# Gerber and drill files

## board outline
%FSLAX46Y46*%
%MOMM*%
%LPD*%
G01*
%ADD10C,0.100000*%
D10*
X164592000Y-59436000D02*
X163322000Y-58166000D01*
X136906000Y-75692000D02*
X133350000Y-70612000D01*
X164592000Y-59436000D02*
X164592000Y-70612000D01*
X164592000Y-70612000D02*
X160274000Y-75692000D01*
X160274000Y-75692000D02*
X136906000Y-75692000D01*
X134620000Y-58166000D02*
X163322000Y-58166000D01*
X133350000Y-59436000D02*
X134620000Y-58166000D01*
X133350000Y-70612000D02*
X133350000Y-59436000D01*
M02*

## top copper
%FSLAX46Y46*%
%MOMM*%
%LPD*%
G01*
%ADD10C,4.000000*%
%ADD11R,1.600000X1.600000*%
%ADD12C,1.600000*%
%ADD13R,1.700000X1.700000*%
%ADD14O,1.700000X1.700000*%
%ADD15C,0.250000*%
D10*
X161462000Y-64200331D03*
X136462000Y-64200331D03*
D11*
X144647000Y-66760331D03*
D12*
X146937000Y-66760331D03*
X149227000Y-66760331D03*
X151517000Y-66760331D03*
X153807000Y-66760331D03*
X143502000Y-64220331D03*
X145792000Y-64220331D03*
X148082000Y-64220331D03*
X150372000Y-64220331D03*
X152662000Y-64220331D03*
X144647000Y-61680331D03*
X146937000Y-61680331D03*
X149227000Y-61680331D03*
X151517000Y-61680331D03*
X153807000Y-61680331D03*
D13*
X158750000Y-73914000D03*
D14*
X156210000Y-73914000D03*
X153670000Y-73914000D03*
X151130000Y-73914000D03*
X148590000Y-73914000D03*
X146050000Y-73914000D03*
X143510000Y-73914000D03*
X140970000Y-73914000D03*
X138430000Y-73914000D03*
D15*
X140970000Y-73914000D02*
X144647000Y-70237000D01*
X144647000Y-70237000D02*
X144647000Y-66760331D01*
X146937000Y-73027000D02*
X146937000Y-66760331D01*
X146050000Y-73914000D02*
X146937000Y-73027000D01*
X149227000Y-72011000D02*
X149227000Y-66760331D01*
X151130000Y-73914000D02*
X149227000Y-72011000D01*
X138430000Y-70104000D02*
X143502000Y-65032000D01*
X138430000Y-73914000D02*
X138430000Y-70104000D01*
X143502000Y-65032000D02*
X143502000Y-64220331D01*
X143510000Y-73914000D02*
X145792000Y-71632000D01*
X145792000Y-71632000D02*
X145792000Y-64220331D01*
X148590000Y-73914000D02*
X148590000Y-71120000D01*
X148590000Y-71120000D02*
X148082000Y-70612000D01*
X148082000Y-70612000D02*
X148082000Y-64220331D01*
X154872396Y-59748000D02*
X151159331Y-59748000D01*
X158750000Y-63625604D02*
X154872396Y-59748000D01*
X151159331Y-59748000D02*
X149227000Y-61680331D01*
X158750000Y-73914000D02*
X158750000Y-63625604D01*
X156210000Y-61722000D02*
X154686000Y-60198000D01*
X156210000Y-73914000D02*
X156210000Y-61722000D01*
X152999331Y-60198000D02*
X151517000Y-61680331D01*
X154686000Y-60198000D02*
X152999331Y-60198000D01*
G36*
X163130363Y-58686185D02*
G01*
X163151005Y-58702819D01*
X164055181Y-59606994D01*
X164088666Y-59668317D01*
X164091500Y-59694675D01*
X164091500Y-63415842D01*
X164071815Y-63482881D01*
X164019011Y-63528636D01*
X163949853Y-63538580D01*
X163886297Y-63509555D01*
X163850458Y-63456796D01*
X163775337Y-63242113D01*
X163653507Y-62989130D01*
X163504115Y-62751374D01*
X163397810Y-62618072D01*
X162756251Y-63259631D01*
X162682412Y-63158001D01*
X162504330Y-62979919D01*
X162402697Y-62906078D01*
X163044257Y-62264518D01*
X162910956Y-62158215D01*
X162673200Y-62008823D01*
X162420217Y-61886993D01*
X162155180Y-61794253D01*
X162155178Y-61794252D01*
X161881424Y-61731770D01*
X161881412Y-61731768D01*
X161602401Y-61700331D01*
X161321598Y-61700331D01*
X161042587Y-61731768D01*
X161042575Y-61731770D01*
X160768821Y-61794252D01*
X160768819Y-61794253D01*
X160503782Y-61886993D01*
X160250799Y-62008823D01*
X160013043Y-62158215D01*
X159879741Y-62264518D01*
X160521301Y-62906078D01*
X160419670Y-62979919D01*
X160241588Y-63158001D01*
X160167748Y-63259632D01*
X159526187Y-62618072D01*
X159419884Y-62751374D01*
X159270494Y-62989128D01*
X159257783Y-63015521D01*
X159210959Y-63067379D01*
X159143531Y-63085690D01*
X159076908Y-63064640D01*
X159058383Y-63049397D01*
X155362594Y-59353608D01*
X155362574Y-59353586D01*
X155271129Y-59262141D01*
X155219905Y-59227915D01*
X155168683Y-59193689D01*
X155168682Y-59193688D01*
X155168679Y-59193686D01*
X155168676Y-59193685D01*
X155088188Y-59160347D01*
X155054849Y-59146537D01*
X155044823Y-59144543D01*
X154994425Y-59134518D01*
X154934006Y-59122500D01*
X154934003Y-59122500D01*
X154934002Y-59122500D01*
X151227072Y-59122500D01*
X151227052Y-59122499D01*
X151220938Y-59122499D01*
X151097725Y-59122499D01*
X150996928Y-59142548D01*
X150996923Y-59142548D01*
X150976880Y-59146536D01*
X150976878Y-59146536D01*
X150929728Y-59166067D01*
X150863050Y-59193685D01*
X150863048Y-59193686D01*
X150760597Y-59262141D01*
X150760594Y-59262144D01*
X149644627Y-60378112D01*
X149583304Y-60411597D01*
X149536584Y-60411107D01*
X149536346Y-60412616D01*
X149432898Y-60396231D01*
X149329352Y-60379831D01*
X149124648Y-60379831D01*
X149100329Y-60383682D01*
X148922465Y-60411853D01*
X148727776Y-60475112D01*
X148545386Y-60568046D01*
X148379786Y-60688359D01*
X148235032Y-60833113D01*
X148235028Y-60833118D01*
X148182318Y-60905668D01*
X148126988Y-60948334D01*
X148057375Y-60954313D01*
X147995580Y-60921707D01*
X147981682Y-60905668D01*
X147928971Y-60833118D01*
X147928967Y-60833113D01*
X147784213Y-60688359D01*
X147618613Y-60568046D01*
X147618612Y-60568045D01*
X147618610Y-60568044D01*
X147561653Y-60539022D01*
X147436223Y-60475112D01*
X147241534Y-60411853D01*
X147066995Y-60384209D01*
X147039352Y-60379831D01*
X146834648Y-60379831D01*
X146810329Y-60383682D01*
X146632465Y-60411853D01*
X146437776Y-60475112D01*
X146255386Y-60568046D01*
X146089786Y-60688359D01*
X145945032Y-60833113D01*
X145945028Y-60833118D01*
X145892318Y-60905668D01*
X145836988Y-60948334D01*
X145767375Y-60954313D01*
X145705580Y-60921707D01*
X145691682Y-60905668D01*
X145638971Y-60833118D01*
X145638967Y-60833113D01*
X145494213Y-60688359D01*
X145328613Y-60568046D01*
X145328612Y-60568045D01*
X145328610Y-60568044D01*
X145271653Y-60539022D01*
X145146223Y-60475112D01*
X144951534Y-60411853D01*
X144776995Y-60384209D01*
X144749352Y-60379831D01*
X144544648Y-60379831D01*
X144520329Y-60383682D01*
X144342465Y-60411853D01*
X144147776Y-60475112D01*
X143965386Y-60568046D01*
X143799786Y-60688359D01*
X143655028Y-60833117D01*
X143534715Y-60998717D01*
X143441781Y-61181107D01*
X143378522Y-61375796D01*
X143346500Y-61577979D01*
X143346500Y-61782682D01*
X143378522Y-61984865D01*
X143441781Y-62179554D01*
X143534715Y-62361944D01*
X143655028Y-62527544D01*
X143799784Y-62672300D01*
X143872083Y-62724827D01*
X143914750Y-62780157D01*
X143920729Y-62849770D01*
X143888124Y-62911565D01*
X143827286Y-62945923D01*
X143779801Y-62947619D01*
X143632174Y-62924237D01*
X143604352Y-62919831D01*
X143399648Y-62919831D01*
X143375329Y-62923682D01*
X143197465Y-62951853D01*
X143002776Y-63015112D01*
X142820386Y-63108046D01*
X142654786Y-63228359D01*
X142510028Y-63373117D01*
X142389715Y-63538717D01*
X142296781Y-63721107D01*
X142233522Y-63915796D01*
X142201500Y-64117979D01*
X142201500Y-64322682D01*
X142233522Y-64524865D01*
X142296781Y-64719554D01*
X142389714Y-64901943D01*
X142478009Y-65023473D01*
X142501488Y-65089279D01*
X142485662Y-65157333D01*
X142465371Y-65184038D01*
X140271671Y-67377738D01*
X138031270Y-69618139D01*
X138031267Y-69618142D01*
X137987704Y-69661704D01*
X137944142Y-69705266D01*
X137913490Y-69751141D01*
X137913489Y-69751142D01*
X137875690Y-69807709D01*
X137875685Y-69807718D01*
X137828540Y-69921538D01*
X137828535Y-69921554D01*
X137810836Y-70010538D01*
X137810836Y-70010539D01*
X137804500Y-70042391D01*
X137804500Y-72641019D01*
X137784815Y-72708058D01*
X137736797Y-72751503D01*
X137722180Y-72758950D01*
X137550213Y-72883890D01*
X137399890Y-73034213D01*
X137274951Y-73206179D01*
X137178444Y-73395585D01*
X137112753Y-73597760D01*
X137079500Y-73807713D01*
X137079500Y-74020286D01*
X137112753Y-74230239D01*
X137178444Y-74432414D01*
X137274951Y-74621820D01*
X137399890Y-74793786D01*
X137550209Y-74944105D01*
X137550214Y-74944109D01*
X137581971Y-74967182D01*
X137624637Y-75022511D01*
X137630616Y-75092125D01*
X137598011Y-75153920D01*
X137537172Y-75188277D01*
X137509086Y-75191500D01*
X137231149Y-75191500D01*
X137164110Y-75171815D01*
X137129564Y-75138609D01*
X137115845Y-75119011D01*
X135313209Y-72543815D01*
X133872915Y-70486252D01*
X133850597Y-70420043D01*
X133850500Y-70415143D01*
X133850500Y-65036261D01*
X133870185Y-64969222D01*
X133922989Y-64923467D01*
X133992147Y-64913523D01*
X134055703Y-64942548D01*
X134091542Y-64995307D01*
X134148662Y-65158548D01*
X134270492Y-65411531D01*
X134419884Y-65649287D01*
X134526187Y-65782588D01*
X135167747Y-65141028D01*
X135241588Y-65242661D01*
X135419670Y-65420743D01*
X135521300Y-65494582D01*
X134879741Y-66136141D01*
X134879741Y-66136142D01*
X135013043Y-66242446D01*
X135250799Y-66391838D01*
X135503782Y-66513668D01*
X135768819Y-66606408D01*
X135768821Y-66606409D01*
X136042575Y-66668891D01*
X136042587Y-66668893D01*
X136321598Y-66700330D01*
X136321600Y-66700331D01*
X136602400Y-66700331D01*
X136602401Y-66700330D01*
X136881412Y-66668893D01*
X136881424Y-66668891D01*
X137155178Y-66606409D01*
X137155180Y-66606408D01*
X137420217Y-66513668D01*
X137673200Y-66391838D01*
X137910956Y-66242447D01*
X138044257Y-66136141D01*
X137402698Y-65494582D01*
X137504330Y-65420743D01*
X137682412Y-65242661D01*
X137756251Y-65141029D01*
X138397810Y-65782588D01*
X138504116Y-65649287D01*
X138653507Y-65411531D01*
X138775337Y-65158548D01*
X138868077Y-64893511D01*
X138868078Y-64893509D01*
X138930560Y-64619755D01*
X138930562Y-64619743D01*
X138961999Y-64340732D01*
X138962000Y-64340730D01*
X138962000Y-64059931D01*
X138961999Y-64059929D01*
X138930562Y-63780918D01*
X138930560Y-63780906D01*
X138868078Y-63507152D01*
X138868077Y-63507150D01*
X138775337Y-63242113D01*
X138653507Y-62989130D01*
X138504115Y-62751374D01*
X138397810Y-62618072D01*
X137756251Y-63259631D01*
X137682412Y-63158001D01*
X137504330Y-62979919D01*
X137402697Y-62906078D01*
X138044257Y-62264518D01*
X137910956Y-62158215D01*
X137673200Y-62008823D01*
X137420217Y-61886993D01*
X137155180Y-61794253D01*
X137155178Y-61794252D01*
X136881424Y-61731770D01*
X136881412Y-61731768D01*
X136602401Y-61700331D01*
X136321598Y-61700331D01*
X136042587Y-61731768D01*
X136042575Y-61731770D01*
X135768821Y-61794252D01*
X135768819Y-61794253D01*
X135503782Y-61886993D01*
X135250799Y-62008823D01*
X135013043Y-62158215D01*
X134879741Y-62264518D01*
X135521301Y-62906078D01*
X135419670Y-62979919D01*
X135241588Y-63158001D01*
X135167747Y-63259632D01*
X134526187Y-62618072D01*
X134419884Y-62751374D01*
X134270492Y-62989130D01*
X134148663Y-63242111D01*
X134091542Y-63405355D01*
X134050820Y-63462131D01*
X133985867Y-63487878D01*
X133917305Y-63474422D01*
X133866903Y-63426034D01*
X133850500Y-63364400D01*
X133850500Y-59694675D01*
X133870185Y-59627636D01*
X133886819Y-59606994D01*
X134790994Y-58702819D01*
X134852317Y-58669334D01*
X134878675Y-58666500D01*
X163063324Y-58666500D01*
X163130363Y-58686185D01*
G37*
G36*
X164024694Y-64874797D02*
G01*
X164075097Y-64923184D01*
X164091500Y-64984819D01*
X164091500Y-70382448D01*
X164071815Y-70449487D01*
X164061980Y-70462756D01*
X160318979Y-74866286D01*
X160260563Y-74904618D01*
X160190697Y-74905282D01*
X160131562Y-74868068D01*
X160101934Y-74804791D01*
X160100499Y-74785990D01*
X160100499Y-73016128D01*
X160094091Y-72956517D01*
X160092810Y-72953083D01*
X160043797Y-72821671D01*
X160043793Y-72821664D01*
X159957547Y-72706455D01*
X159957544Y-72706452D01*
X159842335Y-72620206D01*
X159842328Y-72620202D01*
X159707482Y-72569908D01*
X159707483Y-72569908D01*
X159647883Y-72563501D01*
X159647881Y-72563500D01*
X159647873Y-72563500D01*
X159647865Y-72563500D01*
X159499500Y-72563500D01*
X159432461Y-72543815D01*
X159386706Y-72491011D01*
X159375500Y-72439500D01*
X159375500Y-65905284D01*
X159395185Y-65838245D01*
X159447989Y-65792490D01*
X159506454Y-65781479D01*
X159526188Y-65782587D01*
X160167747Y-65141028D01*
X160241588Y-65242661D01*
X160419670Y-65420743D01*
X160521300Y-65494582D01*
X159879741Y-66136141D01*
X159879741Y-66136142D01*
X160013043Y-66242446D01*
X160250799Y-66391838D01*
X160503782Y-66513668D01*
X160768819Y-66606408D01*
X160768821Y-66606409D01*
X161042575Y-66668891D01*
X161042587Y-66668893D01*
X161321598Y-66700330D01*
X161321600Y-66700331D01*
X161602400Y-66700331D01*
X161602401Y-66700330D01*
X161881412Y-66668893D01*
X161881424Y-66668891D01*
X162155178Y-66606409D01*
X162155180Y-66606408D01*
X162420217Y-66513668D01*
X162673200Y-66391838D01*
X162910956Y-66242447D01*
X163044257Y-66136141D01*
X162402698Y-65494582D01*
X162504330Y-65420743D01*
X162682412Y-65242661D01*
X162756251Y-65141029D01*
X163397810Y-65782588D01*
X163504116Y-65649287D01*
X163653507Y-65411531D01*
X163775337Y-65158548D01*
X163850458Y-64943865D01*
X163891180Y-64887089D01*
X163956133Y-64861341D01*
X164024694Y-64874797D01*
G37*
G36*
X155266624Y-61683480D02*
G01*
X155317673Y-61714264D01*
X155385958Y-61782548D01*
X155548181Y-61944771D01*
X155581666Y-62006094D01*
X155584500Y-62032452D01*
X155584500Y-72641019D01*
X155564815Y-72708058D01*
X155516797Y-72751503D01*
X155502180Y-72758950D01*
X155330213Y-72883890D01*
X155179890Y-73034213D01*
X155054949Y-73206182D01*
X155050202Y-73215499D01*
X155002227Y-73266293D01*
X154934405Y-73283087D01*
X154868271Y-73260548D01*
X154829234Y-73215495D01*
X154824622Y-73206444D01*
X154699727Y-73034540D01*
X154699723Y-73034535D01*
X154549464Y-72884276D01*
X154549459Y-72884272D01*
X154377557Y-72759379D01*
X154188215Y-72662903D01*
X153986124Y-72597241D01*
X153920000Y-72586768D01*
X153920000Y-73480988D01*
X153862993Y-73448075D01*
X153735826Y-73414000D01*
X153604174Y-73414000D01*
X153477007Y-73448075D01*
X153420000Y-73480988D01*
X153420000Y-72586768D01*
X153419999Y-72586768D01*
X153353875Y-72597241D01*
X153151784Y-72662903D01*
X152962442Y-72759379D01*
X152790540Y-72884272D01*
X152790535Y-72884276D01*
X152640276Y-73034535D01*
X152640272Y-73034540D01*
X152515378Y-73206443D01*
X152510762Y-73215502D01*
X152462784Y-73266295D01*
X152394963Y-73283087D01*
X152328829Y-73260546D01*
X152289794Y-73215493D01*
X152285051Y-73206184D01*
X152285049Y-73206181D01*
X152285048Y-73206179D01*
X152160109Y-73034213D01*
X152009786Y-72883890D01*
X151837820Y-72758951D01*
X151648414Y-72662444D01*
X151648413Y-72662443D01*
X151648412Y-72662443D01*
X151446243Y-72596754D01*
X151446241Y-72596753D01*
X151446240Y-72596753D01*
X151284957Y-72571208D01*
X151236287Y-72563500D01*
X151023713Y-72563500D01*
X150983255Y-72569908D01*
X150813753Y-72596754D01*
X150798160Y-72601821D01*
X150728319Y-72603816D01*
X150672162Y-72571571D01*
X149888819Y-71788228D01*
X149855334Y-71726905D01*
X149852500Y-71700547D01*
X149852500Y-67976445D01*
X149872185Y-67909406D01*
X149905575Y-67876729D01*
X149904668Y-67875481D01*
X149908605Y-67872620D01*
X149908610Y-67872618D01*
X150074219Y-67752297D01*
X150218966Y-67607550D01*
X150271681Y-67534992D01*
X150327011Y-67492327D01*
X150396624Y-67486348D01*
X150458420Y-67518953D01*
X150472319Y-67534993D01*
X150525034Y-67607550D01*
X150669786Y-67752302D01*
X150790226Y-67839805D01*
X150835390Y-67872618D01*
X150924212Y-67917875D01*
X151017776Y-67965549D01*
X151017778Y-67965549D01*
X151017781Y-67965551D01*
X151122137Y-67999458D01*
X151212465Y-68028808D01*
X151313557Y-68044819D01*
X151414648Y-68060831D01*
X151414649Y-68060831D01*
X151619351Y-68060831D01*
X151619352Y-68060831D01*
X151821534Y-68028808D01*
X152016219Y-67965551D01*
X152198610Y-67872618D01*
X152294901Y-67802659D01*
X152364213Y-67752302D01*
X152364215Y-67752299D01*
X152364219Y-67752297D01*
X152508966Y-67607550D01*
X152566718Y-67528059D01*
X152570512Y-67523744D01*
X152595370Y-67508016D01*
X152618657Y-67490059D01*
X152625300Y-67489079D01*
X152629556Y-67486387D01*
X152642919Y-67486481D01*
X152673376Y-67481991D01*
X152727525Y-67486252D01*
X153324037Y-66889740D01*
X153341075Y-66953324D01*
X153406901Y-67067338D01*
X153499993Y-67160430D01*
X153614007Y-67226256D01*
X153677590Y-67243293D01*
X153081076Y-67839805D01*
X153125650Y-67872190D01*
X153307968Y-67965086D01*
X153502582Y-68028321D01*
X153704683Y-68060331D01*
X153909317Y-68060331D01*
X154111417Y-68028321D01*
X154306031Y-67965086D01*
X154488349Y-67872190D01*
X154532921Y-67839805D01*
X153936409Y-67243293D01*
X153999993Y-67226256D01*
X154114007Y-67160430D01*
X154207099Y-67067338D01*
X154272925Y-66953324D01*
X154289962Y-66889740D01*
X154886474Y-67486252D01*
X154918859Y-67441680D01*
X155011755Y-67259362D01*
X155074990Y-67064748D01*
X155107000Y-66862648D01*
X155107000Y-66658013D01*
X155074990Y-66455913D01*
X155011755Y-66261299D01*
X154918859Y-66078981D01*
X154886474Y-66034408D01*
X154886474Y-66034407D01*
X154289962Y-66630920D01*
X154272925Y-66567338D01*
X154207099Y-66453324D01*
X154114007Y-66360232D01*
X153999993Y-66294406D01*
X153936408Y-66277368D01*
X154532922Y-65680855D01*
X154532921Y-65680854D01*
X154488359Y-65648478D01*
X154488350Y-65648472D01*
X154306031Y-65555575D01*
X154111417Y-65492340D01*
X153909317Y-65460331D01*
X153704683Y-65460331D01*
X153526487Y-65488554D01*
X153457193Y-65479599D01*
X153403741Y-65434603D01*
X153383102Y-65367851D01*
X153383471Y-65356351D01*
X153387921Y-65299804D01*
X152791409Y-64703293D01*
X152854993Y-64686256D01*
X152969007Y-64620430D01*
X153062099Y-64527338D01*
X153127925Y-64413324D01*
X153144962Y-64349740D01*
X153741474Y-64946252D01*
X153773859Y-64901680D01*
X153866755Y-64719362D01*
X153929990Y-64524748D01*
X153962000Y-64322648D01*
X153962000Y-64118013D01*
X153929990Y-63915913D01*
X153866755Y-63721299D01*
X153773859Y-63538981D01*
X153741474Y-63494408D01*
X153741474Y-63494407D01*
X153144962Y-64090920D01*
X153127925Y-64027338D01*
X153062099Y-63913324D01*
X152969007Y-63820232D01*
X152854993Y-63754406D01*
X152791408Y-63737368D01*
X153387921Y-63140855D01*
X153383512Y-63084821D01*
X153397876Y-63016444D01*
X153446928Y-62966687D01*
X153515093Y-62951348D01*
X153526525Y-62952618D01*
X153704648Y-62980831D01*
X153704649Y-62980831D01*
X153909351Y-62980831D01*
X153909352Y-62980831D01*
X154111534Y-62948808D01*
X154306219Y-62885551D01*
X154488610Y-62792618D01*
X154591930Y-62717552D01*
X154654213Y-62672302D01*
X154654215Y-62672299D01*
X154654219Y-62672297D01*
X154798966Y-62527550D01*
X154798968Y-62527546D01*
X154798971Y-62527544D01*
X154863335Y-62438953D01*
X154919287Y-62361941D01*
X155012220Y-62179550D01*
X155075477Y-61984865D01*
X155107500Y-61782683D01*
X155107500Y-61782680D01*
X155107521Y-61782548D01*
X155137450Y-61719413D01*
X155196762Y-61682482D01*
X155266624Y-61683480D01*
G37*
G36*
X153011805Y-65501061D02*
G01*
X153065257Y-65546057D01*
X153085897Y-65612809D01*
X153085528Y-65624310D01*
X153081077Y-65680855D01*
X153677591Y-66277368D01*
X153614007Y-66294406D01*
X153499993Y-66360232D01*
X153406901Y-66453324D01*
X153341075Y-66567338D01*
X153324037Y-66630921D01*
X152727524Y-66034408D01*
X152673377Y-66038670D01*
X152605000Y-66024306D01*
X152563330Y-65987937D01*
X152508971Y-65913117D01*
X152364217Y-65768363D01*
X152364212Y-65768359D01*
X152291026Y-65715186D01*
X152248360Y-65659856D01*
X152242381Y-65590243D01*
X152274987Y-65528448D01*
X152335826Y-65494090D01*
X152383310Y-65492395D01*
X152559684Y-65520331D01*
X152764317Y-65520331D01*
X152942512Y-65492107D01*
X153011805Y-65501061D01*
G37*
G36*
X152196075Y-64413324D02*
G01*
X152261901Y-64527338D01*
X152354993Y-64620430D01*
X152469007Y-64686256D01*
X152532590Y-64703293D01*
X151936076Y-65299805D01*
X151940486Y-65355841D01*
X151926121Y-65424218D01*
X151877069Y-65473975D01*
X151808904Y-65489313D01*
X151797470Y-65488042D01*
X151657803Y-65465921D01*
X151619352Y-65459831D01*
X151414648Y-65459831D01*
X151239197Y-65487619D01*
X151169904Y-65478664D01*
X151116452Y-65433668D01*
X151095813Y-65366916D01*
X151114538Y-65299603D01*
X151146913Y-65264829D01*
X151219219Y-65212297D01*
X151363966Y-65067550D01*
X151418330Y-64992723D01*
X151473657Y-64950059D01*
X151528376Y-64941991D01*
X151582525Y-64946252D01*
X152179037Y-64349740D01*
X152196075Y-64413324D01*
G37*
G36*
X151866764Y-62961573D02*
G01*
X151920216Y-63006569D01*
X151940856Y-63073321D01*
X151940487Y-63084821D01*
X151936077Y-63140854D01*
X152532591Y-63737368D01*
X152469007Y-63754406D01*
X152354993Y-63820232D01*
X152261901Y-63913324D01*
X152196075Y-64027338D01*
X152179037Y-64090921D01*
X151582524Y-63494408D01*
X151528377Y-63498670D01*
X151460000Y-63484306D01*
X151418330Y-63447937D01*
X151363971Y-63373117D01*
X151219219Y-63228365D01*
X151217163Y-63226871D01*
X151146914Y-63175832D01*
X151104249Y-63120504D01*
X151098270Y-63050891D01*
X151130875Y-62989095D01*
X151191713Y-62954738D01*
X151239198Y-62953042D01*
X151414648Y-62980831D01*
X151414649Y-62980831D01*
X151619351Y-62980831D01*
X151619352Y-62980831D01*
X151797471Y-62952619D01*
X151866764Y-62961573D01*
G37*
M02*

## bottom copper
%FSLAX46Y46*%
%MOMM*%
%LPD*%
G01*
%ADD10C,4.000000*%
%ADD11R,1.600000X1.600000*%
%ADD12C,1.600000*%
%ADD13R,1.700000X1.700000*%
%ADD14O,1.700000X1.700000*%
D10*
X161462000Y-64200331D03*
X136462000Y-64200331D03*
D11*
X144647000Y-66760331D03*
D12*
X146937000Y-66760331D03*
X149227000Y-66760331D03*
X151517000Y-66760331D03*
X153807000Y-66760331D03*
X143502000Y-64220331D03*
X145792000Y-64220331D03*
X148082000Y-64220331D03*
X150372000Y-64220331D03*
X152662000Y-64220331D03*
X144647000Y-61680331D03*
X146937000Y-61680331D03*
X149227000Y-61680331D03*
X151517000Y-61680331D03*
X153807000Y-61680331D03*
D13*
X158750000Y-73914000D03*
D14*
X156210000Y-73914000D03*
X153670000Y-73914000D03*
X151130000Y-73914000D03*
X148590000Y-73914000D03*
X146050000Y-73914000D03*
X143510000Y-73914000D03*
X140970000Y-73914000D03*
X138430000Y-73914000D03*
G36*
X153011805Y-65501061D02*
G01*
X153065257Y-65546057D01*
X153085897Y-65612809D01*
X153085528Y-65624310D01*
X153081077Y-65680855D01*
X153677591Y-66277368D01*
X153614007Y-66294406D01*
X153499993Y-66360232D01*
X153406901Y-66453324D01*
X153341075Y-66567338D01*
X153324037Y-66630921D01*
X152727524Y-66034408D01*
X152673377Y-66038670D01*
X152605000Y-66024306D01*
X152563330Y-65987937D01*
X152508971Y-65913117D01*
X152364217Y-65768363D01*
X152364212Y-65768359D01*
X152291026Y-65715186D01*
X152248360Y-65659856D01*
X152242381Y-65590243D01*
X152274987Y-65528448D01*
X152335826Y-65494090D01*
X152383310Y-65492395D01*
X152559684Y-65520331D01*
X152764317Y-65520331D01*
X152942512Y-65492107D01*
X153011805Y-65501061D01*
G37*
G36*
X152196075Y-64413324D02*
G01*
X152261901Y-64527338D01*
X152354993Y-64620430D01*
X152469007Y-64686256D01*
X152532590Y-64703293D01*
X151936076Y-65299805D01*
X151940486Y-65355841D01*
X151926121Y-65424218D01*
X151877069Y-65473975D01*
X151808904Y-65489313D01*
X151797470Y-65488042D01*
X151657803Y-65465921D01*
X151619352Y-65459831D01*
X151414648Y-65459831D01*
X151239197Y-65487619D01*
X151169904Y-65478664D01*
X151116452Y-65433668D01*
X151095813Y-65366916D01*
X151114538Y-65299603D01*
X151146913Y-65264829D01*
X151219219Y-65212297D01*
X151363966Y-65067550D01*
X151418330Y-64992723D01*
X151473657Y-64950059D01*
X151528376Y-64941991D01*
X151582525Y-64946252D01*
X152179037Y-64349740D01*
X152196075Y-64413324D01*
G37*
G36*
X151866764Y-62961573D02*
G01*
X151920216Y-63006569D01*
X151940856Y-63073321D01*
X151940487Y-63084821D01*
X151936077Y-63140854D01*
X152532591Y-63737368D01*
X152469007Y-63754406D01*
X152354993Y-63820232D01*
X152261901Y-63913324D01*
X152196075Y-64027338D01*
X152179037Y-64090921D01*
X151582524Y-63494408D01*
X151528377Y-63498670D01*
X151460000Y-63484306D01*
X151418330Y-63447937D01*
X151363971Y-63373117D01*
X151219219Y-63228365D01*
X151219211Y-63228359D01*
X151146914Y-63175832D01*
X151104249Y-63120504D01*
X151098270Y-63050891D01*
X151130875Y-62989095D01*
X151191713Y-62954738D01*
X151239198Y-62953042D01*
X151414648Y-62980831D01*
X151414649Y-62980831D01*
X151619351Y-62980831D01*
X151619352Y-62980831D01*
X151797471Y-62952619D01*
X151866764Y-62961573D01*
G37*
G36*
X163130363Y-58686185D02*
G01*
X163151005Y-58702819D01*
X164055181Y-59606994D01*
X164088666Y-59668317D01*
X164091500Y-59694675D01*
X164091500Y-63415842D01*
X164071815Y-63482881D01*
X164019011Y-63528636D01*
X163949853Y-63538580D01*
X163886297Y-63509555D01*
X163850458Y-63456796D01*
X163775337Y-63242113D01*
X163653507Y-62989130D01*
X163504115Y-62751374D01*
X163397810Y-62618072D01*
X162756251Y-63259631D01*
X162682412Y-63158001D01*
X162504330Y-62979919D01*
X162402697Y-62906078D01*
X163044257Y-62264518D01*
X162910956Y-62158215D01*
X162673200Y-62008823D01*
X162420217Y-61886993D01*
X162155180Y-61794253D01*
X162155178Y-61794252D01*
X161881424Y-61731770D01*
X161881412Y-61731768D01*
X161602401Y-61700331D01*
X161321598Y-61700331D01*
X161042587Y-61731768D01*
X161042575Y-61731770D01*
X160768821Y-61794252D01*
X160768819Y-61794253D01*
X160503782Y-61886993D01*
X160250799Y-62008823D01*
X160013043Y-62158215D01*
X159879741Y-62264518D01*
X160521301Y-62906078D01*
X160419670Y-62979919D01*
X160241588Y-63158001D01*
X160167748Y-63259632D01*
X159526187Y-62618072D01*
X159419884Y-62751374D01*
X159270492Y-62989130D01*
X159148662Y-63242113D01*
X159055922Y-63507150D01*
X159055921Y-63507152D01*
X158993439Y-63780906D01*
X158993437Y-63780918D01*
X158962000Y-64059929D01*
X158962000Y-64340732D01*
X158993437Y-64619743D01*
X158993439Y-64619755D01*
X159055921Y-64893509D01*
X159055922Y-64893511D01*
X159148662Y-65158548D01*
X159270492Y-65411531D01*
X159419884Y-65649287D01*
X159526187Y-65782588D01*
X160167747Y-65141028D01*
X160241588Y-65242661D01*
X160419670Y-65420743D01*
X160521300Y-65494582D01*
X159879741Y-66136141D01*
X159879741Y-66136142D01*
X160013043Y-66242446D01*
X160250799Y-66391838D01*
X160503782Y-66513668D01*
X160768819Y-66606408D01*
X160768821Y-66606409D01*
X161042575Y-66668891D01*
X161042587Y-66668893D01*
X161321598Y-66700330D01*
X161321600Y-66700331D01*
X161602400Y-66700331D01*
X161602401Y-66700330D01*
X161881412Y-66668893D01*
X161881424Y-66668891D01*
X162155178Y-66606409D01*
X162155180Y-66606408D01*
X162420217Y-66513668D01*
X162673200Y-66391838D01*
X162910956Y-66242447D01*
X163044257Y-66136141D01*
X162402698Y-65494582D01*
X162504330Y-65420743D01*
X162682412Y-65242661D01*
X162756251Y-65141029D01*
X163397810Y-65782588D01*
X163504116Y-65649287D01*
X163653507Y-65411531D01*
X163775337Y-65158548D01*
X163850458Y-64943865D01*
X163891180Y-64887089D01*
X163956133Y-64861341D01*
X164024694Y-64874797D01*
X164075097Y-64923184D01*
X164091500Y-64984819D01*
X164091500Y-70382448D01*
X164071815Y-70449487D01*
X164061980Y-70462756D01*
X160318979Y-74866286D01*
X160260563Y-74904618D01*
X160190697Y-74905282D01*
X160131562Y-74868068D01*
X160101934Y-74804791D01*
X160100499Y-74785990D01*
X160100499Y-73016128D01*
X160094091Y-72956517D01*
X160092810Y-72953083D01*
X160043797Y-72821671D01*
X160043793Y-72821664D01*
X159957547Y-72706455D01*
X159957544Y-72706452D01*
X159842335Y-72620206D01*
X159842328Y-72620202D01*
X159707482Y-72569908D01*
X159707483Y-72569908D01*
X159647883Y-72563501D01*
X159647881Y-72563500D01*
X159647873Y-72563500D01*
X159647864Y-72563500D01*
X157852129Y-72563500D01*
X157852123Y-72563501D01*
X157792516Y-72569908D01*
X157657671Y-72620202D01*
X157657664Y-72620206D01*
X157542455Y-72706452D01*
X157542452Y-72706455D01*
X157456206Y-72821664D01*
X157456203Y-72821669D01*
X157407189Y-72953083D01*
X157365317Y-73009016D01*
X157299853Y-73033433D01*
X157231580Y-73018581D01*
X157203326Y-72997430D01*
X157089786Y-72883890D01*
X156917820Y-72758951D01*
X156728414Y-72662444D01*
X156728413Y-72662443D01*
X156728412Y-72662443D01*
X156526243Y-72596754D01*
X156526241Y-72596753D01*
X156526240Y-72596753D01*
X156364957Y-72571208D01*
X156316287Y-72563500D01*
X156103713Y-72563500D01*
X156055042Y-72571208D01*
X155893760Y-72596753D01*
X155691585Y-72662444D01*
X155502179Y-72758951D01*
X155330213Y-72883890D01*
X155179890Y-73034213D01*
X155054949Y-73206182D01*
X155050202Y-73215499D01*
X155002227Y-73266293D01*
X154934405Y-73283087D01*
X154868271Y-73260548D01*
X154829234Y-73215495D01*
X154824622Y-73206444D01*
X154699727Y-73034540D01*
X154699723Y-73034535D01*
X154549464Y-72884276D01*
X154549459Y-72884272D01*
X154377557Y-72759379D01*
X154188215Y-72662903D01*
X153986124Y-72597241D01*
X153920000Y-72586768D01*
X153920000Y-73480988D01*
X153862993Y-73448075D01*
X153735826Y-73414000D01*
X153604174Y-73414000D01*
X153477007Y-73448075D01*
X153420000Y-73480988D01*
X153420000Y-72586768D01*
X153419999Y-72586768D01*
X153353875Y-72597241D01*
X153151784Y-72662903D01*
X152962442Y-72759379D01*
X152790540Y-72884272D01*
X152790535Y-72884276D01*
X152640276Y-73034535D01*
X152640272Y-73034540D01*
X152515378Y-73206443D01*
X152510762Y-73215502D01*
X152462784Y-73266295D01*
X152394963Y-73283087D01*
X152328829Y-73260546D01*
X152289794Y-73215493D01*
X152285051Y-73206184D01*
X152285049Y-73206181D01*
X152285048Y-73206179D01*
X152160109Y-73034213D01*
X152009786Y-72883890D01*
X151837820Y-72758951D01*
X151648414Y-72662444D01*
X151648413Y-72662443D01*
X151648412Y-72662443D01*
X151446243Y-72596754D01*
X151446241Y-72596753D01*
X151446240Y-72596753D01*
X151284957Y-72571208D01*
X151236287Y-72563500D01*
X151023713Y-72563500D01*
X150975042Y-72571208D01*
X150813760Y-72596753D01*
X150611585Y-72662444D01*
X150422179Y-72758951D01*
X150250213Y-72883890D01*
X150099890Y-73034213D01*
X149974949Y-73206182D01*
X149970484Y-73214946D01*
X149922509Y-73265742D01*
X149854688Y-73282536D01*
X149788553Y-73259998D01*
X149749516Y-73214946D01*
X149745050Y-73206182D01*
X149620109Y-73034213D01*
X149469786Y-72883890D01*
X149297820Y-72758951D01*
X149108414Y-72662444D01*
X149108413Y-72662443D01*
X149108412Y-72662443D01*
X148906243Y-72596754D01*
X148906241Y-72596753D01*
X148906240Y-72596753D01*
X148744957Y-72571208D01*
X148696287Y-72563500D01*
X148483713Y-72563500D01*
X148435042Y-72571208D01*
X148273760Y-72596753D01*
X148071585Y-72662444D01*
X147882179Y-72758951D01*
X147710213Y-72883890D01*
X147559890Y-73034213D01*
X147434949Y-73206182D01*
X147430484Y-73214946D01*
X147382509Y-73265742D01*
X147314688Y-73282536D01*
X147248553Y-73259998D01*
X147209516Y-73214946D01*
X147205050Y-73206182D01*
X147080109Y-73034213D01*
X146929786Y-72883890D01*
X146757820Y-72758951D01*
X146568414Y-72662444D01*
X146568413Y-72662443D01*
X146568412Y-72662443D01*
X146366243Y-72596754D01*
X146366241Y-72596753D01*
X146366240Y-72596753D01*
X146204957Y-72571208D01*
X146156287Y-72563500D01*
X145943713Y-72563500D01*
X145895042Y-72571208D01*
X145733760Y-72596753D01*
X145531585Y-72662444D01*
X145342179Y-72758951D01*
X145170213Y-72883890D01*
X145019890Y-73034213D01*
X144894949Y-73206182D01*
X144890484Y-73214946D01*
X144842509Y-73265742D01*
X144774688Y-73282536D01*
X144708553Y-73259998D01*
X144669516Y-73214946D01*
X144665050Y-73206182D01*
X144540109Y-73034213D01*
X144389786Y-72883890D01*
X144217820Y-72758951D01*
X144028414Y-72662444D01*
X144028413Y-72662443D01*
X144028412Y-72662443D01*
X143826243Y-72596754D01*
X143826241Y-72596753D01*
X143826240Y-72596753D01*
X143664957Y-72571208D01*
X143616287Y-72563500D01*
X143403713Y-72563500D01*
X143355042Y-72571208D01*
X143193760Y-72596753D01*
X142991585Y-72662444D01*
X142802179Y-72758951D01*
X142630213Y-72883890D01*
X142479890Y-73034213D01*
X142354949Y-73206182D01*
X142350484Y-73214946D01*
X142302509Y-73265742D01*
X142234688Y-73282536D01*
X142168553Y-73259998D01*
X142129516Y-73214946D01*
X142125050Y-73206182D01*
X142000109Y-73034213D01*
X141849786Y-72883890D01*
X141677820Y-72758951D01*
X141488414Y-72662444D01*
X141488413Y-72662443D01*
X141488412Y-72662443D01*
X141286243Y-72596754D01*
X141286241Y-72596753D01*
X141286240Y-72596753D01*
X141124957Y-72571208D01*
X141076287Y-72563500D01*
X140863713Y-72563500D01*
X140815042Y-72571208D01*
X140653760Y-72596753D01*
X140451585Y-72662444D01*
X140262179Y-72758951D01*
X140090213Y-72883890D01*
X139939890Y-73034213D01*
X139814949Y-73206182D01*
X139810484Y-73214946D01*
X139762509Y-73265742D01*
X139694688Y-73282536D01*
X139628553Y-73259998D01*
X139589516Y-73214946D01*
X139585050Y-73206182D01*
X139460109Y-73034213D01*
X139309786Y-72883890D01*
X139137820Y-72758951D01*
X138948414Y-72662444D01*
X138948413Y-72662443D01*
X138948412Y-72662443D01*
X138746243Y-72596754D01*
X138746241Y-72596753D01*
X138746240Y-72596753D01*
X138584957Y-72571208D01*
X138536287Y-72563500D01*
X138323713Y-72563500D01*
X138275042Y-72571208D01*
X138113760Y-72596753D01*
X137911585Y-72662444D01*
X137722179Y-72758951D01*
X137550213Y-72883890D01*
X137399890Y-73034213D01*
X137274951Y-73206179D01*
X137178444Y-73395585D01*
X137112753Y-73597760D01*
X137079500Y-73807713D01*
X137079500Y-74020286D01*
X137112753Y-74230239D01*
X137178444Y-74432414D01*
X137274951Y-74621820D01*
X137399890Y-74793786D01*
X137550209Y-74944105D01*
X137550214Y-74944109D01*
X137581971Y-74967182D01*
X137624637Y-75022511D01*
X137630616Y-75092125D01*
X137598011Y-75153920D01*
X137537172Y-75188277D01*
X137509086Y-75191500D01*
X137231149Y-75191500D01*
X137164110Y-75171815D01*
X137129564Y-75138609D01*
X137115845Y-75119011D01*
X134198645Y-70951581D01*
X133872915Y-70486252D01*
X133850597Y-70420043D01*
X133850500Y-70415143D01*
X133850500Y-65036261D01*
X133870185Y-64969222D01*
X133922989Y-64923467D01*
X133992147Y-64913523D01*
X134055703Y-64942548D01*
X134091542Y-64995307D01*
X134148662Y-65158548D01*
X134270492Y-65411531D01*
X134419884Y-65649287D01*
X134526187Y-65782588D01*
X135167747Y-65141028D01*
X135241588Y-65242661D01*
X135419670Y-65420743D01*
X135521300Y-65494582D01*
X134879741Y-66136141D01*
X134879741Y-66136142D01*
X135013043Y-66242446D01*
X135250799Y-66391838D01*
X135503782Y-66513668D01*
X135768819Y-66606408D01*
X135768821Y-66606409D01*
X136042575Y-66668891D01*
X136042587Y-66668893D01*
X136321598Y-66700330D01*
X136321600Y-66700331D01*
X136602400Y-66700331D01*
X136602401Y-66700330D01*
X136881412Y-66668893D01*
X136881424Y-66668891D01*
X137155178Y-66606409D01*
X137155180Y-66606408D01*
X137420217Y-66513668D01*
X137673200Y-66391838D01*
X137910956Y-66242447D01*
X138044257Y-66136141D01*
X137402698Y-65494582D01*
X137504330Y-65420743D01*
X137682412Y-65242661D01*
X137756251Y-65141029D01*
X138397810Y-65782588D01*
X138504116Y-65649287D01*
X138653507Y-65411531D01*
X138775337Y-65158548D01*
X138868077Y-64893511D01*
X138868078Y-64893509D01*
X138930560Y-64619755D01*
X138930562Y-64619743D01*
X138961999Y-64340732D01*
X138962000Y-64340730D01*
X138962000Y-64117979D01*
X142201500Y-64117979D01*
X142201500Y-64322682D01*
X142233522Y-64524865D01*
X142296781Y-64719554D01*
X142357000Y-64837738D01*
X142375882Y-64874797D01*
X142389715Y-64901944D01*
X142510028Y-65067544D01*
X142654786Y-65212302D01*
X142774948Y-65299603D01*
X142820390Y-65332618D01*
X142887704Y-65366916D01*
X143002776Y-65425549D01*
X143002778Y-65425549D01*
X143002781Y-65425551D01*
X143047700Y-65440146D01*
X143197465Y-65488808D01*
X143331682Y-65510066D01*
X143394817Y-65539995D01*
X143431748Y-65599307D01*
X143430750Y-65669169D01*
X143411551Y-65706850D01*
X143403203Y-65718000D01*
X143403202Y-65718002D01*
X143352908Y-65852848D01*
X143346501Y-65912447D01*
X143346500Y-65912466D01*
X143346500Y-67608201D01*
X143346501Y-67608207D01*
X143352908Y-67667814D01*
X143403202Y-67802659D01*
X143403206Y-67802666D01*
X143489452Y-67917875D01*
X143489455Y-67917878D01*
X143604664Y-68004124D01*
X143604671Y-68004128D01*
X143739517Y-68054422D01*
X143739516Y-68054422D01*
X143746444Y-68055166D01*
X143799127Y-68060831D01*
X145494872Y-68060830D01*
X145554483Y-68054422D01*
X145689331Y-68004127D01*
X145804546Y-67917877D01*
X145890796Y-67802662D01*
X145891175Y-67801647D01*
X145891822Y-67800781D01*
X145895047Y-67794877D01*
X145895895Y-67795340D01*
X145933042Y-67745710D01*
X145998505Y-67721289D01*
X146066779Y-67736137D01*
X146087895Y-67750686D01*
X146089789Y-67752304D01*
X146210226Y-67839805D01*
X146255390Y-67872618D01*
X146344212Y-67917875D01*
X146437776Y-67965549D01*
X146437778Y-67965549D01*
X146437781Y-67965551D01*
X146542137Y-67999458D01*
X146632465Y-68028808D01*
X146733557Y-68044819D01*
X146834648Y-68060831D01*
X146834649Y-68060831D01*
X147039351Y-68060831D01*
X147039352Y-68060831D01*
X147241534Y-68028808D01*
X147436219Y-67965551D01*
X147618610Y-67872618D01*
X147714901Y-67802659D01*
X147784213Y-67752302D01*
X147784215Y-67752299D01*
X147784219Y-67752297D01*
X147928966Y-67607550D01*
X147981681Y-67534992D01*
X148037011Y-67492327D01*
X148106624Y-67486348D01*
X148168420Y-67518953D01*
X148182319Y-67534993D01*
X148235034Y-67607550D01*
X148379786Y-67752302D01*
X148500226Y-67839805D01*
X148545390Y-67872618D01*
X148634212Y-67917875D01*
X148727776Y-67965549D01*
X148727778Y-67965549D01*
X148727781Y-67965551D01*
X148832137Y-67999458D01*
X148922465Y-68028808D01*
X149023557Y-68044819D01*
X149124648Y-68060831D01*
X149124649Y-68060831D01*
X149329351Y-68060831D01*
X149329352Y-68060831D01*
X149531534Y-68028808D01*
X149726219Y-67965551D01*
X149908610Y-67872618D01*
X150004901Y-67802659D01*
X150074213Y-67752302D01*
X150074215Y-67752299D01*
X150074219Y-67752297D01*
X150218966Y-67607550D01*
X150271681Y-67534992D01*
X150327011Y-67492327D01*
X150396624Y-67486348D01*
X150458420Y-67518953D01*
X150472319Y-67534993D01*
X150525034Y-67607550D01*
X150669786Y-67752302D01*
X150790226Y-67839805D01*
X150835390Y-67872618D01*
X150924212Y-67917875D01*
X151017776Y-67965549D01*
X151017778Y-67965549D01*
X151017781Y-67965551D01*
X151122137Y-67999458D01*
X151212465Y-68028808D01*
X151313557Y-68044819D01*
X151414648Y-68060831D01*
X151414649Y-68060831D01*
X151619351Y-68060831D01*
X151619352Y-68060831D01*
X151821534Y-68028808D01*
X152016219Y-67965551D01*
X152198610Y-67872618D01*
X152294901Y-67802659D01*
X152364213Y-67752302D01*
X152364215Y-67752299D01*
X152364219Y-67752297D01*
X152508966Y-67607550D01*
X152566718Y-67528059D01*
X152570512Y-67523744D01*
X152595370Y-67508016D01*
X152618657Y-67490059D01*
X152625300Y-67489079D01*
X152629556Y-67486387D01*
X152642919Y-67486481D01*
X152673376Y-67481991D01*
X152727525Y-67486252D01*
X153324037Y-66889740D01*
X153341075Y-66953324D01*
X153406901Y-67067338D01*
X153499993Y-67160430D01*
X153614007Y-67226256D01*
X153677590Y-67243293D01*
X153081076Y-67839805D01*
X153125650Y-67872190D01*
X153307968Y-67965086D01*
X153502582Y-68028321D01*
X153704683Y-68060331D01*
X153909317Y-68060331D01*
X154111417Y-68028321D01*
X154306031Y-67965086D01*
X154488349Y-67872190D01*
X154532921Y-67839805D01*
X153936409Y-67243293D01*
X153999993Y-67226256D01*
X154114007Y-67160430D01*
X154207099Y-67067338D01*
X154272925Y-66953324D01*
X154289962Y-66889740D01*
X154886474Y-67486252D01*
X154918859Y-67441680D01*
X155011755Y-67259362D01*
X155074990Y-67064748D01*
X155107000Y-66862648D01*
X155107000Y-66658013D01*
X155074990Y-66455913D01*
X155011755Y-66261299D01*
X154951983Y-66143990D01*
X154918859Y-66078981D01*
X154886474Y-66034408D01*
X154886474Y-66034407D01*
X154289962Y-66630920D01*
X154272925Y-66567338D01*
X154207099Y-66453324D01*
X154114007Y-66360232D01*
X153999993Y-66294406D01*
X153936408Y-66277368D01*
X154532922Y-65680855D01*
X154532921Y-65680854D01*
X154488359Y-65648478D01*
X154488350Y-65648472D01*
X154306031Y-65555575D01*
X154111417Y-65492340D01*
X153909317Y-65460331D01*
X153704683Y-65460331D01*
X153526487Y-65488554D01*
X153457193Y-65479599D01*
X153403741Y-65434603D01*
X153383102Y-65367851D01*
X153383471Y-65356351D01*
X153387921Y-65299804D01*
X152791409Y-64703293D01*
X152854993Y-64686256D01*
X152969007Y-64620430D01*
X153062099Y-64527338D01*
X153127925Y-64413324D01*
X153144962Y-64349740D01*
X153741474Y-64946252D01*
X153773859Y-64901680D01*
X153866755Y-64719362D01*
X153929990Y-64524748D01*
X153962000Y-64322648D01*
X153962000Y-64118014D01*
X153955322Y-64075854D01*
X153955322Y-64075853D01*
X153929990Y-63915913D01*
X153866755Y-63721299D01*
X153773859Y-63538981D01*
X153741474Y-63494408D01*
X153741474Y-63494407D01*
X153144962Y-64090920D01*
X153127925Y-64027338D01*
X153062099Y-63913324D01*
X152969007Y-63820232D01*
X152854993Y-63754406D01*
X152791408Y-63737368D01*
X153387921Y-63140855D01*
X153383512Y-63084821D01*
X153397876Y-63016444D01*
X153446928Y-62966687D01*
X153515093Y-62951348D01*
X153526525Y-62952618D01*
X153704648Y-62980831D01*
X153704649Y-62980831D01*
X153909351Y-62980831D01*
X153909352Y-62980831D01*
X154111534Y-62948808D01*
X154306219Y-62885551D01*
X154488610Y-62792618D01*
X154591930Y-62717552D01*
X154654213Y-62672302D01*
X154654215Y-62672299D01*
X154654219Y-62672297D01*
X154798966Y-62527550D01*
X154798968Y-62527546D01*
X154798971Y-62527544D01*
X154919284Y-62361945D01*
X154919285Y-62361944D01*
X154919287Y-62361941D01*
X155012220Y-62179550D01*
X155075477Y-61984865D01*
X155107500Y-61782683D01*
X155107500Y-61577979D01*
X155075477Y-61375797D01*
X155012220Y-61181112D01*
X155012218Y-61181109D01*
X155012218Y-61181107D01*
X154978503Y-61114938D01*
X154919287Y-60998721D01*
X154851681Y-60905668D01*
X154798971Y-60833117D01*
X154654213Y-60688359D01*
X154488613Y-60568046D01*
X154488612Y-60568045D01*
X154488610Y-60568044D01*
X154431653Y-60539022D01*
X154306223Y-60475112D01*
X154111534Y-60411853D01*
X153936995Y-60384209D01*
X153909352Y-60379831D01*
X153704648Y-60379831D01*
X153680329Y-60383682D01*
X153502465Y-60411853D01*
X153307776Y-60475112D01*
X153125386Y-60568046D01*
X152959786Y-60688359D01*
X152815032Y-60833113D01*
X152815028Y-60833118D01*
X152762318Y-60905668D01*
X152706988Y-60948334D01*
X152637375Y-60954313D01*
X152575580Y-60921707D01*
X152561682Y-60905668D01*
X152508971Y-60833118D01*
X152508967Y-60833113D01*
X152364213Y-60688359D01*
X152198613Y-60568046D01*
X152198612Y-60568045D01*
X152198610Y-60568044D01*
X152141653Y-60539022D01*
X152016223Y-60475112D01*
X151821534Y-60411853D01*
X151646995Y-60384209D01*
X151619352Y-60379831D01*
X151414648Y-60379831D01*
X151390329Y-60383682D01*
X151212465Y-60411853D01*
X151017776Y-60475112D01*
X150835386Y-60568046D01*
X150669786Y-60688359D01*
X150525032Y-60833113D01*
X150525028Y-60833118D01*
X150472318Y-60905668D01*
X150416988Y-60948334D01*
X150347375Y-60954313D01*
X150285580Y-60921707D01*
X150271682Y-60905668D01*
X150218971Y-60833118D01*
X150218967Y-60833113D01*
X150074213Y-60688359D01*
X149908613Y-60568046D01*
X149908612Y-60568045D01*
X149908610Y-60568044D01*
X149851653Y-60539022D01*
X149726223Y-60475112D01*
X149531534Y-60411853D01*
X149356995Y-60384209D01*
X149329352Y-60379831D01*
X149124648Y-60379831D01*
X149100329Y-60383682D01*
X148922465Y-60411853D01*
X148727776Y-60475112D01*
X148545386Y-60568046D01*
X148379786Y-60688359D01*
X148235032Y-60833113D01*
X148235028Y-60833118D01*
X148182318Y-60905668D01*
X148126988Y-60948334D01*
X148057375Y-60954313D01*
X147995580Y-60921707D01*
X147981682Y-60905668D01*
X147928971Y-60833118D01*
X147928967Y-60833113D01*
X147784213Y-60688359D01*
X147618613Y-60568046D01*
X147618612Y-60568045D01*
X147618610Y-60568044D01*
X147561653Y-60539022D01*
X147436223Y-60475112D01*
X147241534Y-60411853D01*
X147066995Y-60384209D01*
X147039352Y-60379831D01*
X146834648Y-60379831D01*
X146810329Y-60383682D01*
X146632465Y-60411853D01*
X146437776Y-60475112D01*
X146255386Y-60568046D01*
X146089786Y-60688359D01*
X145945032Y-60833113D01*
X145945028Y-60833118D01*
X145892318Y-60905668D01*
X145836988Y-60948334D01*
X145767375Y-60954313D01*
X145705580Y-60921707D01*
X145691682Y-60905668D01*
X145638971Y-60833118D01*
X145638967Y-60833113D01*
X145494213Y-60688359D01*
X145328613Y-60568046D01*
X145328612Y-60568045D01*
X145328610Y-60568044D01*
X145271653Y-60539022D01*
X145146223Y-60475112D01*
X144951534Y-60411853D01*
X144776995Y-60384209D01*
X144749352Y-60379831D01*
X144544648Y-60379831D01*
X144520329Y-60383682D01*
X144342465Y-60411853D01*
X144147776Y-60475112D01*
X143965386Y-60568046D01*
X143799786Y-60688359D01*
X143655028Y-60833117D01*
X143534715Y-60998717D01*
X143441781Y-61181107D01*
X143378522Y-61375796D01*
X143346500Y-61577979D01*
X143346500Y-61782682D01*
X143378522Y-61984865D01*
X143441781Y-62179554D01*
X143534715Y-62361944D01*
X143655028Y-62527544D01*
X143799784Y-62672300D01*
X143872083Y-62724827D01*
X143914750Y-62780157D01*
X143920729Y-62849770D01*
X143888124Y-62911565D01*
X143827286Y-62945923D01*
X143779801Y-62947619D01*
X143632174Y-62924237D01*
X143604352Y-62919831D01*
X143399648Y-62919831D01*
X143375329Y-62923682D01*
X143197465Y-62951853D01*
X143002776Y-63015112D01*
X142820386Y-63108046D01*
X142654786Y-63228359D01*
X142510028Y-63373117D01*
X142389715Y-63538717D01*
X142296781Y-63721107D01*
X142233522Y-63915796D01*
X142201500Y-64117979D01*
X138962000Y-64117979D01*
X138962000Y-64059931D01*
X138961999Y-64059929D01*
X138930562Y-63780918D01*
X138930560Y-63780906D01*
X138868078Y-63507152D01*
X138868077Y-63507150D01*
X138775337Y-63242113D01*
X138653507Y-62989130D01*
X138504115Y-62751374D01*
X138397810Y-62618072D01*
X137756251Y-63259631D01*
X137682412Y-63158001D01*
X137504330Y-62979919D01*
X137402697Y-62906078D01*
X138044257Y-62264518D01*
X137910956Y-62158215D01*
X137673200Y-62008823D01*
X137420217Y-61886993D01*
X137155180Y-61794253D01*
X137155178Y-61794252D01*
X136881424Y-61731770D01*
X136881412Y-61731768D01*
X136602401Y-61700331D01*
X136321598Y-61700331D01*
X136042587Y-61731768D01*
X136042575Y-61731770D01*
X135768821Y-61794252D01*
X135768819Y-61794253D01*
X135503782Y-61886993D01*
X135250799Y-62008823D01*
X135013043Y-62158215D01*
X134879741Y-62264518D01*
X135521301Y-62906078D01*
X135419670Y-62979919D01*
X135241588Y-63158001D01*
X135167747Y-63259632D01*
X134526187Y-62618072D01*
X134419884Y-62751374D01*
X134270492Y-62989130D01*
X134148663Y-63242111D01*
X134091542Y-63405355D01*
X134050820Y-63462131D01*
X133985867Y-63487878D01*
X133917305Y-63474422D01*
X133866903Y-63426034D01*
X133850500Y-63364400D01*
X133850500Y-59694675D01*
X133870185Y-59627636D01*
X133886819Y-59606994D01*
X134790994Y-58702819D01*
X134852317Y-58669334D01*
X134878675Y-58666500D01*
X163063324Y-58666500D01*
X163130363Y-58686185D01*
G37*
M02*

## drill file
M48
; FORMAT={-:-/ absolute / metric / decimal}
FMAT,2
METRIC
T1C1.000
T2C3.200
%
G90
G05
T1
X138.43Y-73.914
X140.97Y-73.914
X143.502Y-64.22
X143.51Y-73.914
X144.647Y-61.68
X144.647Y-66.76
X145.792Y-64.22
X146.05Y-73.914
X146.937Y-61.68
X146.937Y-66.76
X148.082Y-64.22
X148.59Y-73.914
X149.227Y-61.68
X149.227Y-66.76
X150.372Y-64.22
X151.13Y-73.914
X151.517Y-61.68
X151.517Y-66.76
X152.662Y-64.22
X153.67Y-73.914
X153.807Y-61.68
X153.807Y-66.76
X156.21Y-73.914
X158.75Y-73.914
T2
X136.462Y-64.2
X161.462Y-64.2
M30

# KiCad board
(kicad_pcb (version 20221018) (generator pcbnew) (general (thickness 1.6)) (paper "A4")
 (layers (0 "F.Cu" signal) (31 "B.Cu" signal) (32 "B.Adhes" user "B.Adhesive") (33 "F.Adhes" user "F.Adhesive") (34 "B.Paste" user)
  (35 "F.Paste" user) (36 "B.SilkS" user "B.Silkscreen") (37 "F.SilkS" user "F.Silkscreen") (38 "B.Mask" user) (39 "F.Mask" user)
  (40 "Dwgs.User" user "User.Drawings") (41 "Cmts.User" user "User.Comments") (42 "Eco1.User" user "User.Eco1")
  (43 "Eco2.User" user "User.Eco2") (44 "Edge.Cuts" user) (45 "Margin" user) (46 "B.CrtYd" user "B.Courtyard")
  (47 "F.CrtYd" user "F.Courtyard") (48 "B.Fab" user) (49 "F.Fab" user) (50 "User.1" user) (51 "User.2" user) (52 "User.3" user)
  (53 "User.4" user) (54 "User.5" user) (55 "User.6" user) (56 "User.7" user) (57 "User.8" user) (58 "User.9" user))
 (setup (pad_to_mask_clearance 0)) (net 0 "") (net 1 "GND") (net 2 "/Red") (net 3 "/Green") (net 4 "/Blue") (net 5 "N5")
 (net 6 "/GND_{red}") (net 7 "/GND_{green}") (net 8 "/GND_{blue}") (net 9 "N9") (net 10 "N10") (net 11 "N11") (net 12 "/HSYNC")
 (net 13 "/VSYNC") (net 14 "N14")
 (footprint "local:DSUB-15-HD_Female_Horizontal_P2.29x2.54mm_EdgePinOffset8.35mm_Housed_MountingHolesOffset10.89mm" (layer "F.Cu")
  (at 144.647 66.760331 180)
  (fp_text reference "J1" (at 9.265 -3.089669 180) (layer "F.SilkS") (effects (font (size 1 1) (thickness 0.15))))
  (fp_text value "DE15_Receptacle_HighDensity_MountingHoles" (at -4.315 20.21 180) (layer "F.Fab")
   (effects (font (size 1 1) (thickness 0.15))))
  (pad "0" thru_hole circle (at -16.815 2.56 180) (size 4 4) (drill 3.2) (layers "*.Cu" "*.Mask") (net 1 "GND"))
  (pad "0" thru_hole circle (at 8.185 2.56 180) (size 4 4) (drill 3.2) (layers "*.Cu" "*.Mask") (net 1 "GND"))
  (pad "1" thru_hole rect (at 0 0 180) (size 1.6 1.6) (drill 1) (layers "*.Cu" "*.Mask") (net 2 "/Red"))
  (pad "2" thru_hole circle (at -2.29 0 180) (size 1.6 1.6) (drill 1) (layers "*.Cu" "*.Mask") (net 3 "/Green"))
  (pad "3" thru_hole circle (at -4.58 0 180) (size 1.6 1.6) (drill 1) (layers "*.Cu" "*.Mask") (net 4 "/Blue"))
  (pad "4" thru_hole circle (at -6.87 0 180) (size 1.6 1.6) (drill 1) (layers "*.Cu" "*.Mask") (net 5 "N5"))
  (pad "5" thru_hole circle (at -9.16 0 180) (size 1.6 1.6) (drill 1) (layers "*.Cu" "*.Mask") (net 1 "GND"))
  (pad "6" thru_hole circle (at 1.145 2.54 180) (size 1.6 1.6) (drill 1) (layers "*.Cu" "*.Mask") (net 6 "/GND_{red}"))
  (pad "7" thru_hole circle (at -1.145 2.54 180) (size 1.6 1.6) (drill 1) (layers "*.Cu" "*.Mask") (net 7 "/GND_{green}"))
  (pad "8" thru_hole circle (at -3.435 2.54 180) (size 1.6 1.6) (drill 1) (layers "*.Cu" "*.Mask") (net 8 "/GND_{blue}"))
  (pad "9" thru_hole circle (at -5.725 2.54 180) (size 1.6 1.6) (drill 1) (layers "*.Cu" "*.Mask") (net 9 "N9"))
  (pad "10" thru_hole circle (at -8.015 2.54 180) (size 1.6 1.6) (drill 1) (layers "*.Cu" "*.Mask") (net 1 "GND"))
  (pad "11" thru_hole circle (at 0 5.08 180) (size 1.6 1.6) (drill 1) (layers "*.Cu" "*.Mask") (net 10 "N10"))
  (pad "12" thru_hole circle (at -2.29 5.08 180) (size 1.6 1.6) (drill 1) (layers "*.Cu" "*.Mask") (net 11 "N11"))
  (pad "13" thru_hole circle (at -4.58 5.08 180) (size 1.6 1.6) (drill 1) (layers "*.Cu" "*.Mask") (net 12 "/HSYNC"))
  (pad "14" thru_hole circle (at -6.87 5.08 180) (size 1.6 1.6) (drill 1) (layers "*.Cu" "*.Mask") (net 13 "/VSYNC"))
  (pad "15" thru_hole circle (at -9.16 5.08 180) (size 1.6 1.6) (drill 1) (layers "*.Cu" "*.Mask") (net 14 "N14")))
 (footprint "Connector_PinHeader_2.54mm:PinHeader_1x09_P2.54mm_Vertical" (layer "B.Cu") (at 158.75 73.914 90)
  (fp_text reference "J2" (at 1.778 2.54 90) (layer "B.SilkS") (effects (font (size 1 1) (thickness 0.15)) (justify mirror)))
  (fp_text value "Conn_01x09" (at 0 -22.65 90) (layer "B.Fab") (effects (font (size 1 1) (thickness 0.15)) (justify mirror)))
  (pad "1" thru_hole rect (at 0 0 90) (size 1.7 1.7) (drill 1) (layers "*.Cu" "*.Mask") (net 12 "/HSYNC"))
  (pad "2" thru_hole oval (at 0 -2.54 90) (size 1.7 1.7) (drill 1) (layers "*.Cu" "*.Mask") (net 13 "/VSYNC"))
  (pad "3" thru_hole oval (at 0 -5.08 90) (size 1.7 1.7) (drill 1) (layers "*.Cu" "*.Mask") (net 1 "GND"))
  (pad "4" thru_hole oval (at 0 -7.62 90) (size 1.7 1.7) (drill 1) (layers "*.Cu" "*.Mask") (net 4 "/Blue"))
  (pad "5" thru_hole oval (at 0 -10.16 90) (size 1.7 1.7) (drill 1) (layers "*.Cu" "*.Mask") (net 8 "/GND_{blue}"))
  (pad "6" thru_hole oval (at 0 -12.7 90) (size 1.7 1.7) (drill 1) (layers "*.Cu" "*.Mask") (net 3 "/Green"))
  (pad "7" thru_hole oval (at 0 -15.24 90) (size 1.7 1.7) (drill 1) (layers "*.Cu" "*.Mask") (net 7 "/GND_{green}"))
  (pad "8" thru_hole oval (at 0 -17.78 90) (size 1.7 1.7) (drill 1) (layers "*.Cu" "*.Mask") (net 2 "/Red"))
  (pad "9" thru_hole oval (at 0 -20.32 90) (size 1.7 1.7) (drill 1) (layers "*.Cu" "*.Mask") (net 6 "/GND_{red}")))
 (gr_line (start 164.592 59.436) (end 163.322 58.166) (stroke (width 0.1) (type default)) (layer "Edge.Cuts"))
 (gr_line (start 136.906 75.692) (end 133.35 70.612) (stroke (width 0.1) (type default)) (layer "Edge.Cuts"))
 (gr_line (start 164.592 59.436) (end 164.592 70.612) (stroke (width 0.1) (type default)) (layer "Edge.Cuts"))
 (gr_line (start 164.592 70.612) (end 160.274 75.692) (stroke (width 0.1) (type default)) (layer "Edge.Cuts"))
 (gr_line (start 160.274 75.692) (end 136.906 75.692) (stroke (width 0.1) (type default)) (layer "Edge.Cuts"))
 (gr_line (start 134.62 58.166) (end 163.322 58.166) (stroke (width 0.1) (type default)) (layer "Edge.Cuts"))
 (gr_line (start 133.35 59.436) (end 134.62 58.166) (stroke (width 0.1) (type default)) (layer "Edge.Cuts"))
 (gr_line (start 133.35 70.612) (end 133.35 59.436) (stroke (width 0.1) (type default)) (layer "Edge.Cuts"))
 (segment (start 140.97 73.914) (end 144.647 70.237) (width 0.25) (layer "F.Cu") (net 2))
 (segment (start 144.647 70.237) (end 144.647 66.760331) (width 0.25) (layer "F.Cu") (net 2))
 (segment (start 146.937 73.027) (end 146.937 66.760331) (width 0.25) (layer "F.Cu") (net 3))
 (segment (start 146.05 73.914) (end 146.937 73.027) (width 0.25) (layer "F.Cu") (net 3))
 (segment (start 149.227 72.011) (end 149.227 66.760331) (width 0.25) (layer "F.Cu") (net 4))
 (segment (start 151.13 73.914) (end 149.227 72.011) (width 0.25) (layer "F.Cu") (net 4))
 (segment (start 138.43 70.104) (end 143.502 65.032) (width 0.25) (layer "F.Cu") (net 6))
 (segment (start 138.43 73.914) (end 138.43 70.104) (width 0.25) (layer "F.Cu") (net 6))
 (segment (start 143.502 65.032) (end 143.502 64.220331) (width 0.25) (layer "F.Cu") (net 6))
 (segment (start 143.51 73.914) (end 145.792 71.632) (width 0.25) (layer "F.Cu") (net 7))
 (segment (start 145.792 71.632) (end 145.792 64.220331) (width 0.25) (layer "F.Cu") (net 7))
 (segment (start 148.59 73.914) (end 148.59 71.12) (width 0.25) (layer "F.Cu") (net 8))
 (segment (start 148.59 71.12) (end 148.082 70.612) (width 0.25) (layer "F.Cu") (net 8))
 (segment (start 148.082 70.612) (end 148.082 64.220331) (width 0.25) (layer "F.Cu") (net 8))
 (segment (start 154.872396 59.748) (end 151.159331 59.748) (width 0.25) (layer "F.Cu") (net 12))
 (segment (start 158.75 63.625604) (end 154.872396 59.748) (width 0.25) (layer "F.Cu") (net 12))
 (segment (start 151.159331 59.748) (end 149.227 61.680331) (width 0.25) (layer "F.Cu") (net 12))
 (segment (start 158.75 73.914) (end 158.75 63.625604) (width 0.25) (layer "F.Cu") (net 12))
 (segment (start 156.21 61.722) (end 154.686 60.198) (width 0.25) (layer "F.Cu") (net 13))
 (segment (start 156.21 73.914) (end 156.21 61.722) (width 0.25) (layer "F.Cu") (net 13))
 (segment (start 152.999331 60.198) (end 151.517 61.680331) (width 0.25) (layer "F.Cu") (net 13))
 (segment (start 154.686 60.198) (end 152.999331 60.198) (width 0.25) (layer "F.Cu") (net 13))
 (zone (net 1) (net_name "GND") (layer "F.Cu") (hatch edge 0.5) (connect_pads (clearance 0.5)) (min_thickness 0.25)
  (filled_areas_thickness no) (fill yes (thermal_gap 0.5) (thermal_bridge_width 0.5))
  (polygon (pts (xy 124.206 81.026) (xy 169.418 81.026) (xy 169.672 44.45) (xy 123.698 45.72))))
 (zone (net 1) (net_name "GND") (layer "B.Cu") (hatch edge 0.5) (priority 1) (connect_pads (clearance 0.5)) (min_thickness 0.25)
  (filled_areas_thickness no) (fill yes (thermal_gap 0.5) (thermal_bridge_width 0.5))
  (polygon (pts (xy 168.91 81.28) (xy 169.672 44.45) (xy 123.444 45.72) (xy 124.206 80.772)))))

